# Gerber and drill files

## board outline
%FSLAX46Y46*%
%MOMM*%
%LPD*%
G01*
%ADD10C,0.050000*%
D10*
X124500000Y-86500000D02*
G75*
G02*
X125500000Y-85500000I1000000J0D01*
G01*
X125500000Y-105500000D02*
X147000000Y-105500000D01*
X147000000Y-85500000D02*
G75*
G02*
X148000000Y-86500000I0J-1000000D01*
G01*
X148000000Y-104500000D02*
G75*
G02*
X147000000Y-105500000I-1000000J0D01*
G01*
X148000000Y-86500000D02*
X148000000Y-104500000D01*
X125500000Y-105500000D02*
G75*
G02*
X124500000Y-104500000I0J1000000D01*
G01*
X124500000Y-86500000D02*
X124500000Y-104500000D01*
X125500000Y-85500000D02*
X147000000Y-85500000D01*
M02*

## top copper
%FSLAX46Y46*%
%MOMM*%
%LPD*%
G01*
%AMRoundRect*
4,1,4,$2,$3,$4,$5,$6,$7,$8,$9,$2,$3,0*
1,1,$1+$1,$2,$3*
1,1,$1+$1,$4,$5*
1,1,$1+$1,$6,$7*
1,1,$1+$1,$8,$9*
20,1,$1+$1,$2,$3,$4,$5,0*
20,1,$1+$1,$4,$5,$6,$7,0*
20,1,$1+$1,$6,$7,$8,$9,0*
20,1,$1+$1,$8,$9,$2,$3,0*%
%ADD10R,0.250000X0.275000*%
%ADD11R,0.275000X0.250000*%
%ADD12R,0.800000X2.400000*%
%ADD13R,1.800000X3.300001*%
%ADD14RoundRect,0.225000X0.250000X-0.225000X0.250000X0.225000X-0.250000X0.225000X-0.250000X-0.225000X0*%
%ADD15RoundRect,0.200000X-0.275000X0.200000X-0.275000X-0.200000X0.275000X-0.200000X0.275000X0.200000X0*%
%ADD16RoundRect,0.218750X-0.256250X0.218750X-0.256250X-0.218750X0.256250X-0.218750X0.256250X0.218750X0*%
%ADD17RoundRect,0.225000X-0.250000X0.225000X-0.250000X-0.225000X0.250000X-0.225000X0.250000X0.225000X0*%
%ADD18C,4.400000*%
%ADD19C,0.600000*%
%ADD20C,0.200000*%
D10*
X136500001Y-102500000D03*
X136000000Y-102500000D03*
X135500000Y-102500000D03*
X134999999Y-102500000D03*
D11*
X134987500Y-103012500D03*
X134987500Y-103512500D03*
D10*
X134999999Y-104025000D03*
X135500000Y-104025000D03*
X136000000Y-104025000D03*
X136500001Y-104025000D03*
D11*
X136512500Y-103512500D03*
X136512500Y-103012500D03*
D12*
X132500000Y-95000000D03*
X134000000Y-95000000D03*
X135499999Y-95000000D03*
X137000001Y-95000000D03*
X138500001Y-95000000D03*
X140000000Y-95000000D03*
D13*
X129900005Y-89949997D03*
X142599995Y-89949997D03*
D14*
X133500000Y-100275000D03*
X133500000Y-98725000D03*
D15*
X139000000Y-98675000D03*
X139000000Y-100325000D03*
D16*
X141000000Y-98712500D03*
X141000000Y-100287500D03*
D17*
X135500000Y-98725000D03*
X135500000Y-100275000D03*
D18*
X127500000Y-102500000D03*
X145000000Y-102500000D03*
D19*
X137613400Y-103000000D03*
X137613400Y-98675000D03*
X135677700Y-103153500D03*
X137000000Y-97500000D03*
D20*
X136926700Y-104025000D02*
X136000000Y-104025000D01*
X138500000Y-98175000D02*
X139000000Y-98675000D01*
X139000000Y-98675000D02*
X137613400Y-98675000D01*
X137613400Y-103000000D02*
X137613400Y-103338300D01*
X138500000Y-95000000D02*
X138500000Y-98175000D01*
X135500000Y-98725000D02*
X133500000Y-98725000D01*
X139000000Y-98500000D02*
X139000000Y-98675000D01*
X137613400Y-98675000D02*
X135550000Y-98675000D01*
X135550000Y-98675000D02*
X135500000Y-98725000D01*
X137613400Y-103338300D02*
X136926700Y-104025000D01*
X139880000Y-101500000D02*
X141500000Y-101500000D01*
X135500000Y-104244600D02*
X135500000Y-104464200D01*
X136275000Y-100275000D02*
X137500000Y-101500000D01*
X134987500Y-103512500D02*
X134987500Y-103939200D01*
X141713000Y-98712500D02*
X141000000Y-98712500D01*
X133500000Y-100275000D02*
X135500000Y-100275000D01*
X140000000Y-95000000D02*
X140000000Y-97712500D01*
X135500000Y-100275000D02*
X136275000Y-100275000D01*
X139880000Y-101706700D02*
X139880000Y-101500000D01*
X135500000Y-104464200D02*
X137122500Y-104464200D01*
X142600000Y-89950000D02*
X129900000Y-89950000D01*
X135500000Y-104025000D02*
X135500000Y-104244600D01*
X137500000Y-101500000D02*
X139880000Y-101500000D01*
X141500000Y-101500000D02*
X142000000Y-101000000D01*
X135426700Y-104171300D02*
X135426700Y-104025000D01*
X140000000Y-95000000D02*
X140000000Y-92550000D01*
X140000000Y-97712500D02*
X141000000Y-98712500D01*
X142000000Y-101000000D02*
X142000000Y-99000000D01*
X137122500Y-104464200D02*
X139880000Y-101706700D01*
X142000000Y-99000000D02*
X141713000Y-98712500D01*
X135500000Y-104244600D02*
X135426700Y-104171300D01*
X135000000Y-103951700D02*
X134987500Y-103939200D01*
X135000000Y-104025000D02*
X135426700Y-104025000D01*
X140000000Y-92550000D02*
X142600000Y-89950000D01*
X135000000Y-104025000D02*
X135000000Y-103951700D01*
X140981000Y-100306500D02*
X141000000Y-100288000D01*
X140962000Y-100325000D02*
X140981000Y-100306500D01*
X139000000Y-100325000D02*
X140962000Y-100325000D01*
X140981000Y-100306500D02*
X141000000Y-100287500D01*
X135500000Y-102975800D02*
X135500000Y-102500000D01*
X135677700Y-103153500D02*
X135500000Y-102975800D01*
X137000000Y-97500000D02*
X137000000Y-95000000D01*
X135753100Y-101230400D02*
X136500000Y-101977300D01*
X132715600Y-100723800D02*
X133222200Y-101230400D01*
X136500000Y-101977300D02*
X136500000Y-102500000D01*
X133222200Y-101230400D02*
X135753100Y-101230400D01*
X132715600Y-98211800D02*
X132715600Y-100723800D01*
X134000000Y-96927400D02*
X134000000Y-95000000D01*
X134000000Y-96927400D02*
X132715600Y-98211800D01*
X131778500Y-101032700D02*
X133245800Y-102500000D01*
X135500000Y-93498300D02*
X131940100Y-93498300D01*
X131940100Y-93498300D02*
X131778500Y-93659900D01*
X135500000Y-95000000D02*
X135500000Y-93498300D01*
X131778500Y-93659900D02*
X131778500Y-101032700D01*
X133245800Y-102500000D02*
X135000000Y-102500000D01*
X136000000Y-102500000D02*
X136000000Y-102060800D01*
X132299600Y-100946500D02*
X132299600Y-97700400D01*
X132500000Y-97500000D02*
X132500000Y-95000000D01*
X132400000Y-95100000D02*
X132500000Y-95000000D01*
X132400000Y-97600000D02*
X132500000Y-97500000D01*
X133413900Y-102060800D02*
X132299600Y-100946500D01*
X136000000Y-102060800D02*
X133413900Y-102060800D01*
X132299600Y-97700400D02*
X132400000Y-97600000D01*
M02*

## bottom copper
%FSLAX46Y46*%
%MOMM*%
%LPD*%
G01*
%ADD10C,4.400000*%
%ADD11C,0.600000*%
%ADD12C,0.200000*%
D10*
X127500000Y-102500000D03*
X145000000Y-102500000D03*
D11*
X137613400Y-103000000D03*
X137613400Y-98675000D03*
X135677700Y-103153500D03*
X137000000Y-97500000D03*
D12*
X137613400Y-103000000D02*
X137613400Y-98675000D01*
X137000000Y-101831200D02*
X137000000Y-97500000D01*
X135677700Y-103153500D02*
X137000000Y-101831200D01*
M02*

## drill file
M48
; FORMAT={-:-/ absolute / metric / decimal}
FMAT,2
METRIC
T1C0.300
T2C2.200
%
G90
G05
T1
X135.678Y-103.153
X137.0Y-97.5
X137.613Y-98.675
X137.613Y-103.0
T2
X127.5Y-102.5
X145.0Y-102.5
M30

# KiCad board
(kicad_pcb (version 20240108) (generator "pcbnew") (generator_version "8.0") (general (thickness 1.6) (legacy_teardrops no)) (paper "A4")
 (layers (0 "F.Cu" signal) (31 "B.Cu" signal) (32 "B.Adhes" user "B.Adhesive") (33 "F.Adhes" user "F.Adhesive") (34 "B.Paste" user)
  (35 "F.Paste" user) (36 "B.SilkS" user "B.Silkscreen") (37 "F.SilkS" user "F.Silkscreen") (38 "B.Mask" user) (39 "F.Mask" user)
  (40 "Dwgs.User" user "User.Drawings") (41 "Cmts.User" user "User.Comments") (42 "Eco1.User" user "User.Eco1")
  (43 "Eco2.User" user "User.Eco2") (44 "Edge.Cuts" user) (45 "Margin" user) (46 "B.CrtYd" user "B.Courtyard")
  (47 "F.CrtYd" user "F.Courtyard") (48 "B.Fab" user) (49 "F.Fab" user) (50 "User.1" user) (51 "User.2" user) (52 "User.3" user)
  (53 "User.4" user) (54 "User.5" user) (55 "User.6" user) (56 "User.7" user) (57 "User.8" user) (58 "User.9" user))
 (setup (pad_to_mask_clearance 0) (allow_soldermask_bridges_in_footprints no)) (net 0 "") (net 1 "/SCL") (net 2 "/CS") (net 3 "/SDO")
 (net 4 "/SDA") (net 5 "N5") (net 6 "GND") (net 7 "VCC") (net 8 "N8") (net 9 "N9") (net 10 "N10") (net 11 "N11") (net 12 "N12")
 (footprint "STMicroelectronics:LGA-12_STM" (layer "F.Cu") (at 135.75 103.2625 -90)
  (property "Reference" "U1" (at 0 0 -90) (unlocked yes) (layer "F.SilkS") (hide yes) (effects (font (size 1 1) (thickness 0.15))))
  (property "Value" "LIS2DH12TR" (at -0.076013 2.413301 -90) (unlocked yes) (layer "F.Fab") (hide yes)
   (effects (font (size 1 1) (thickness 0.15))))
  (pad "1" smd rect (at -0.7625 -0.750001) (size 0.25 0.275) (layers "F.Cu" "F.Paste" "F.Mask") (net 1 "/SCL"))
  (pad "2" smd rect (at -0.7625 -0.25) (size 0.25 0.275) (layers "F.Cu" "F.Paste" "F.Mask") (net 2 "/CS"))
  (pad "3" smd rect (at -0.7625 0.25) (size 0.25 0.275) (layers "F.Cu" "F.Paste" "F.Mask") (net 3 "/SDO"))
  (pad "4" smd rect (at -0.7625 0.750001) (size 0.25 0.275) (layers "F.Cu" "F.Paste" "F.Mask") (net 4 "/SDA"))
  (pad "5" smd rect (at -0.25 0.7625 270) (size 0.25 0.275) (layers "F.Cu" "F.Paste" "F.Mask") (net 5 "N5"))
  (pad "6" smd rect (at 0.25 0.7625 270) (size 0.25 0.275) (layers "F.Cu" "F.Paste" "F.Mask") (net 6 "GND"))
  (pad "7" smd rect (at 0.7625 0.750001) (size 0.25 0.275) (layers "F.Cu" "F.Paste" "F.Mask") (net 6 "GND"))
  (pad "8" smd rect (at 0.7625 0.25) (size 0.25 0.275) (layers "F.Cu" "F.Paste" "F.Mask") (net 6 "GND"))
  (pad "9" smd rect (at 0.7625 -0.25) (size 0.25 0.275) (layers "F.Cu" "F.Paste" "F.Mask") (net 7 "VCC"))
  (pad "10" smd rect (at 0.7625 -0.750001) (size 0.25 0.275) (layers "F.Cu" "F.Paste" "F.Mask") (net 7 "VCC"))
  (pad "11" smd rect (at 0.25 -0.7625 270) (size 0.25 0.275) (layers "F.Cu" "F.Paste" "F.Mask") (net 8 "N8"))
  (pad "12" smd rect (at -0.25 -0.7625 270) (size 0.25 0.275) (layers "F.Cu" "F.Paste" "F.Mask") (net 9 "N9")))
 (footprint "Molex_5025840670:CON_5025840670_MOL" (layer "F.Cu") (at 132.5 95)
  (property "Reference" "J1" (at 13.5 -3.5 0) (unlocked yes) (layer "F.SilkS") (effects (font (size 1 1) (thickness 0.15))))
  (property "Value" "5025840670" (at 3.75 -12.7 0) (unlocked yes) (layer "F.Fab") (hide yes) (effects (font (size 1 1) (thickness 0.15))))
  (pad "1" smd rect (at 0 0) (size 0.8 2.4) (layers "F.Cu" "F.Paste" "F.Mask") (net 2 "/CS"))
  (pad "2" smd rect (at 1.5 0) (size 0.8 2.4) (layers "F.Cu" "F.Paste" "F.Mask") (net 1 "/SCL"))
  (pad "3" smd rect (at 2.999999 0) (size 0.8 2.4) (layers "F.Cu" "F.Paste" "F.Mask") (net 4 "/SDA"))
  (pad "4" smd rect (at 4.500001 0) (size 0.8 2.4) (layers "F.Cu" "F.Paste" "F.Mask") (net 3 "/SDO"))
  (pad "5" smd rect (at 6.000001 0) (size 0.8 2.4) (layers "F.Cu" "F.Paste" "F.Mask") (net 7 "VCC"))
  (pad "6" smd rect (at 7.5 0) (size 0.8 2.4) (layers "F.Cu" "F.Paste" "F.Mask") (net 6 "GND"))
  (pad "7" smd rect (at -2.599995 -5.050003) (size 1.8 3.300001) (layers "F.Cu" "F.Paste" "F.Mask") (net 6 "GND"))
  (pad "8" smd rect (at 10.099995 -5.050003) (size 1.8 3.300001) (layers "F.Cu" "F.Paste" "F.Mask") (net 6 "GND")))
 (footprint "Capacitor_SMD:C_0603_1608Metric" (layer "F.Cu") (at 133.5 99.5 90)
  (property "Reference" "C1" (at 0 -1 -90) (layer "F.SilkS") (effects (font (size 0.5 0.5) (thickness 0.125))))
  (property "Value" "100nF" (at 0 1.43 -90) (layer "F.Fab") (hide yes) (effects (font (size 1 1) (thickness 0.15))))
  (pad "1" smd roundrect (at -0.775 0 90) (size 0.9 0.95) (layers "F.Cu" "F.Paste" "F.Mask") (roundrect_rratio 0.25) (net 6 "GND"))
  (pad "2" smd roundrect (at 0.775 0 90) (size 0.9 0.95) (layers "F.Cu" "F.Paste" "F.Mask") (roundrect_rratio 0.25) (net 7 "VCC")))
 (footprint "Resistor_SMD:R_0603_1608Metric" (layer "F.Cu") (at 139 99.5 -90)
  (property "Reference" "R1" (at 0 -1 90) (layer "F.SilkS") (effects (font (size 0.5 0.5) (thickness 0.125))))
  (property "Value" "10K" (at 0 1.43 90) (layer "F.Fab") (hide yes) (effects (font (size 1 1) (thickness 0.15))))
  (pad "1" smd roundrect (at -0.825 0 270) (size 0.8 0.95) (layers "F.Cu" "F.Paste" "F.Mask") (roundrect_rratio 0.25) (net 7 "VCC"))
  (pad "2" smd roundrect (at 0.825 0 270) (size 0.8 0.95) (layers "F.Cu" "F.Paste" "F.Mask") (roundrect_rratio 0.25) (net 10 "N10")))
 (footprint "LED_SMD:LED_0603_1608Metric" (layer "F.Cu") (at 141 99.5 -90)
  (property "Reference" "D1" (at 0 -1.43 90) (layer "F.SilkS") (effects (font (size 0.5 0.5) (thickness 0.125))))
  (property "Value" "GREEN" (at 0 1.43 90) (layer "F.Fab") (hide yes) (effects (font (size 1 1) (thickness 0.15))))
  (pad "1" smd roundrect (at -0.7875 0 270) (size 0.875 0.95) (layers "F.Cu" "F.Paste" "F.Mask") (roundrect_rratio 0.25) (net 6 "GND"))
  (pad "2" smd roundrect (at 0.7875 0 270) (size 0.875 0.95) (layers "F.Cu" "F.Paste" "F.Mask") (roundrect_rratio 0.25) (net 10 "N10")))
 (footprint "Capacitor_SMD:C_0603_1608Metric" (layer "F.Cu") (at 135.5 99.5 -90)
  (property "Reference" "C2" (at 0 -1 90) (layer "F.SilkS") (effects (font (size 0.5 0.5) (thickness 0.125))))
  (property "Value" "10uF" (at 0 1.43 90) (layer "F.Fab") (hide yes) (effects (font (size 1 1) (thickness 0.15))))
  (pad "1" smd roundrect (at -0.775 0 270) (size 0.9 0.95) (layers "F.Cu" "F.Paste" "F.Mask") (roundrect_rratio 0.25) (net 7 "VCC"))
  (pad "2" smd roundrect (at 0.775 0 270) (size 0.9 0.95) (layers "F.Cu" "F.Paste" "F.Mask") (roundrect_rratio 0.25) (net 6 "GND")))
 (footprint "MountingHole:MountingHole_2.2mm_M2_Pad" (layer "F.Cu") (at 127.5 102.5)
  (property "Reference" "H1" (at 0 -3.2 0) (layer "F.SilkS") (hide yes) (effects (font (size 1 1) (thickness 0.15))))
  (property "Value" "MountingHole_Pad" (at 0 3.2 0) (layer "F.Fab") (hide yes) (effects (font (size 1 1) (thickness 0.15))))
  (pad "1" thru_hole circle (at 0 0) (size 4.4 4.4) (drill 2.2) (layers "*.Cu" "*.Mask") (remove_unused_layers no) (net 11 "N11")))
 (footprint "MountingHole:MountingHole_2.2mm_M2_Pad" (layer "F.Cu") (at 145 102.5)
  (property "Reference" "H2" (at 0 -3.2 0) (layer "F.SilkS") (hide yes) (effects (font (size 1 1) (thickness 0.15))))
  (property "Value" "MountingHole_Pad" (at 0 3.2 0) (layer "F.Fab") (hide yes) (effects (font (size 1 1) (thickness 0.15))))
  (pad "1" thru_hole circle (at 0 0) (size 4.4 4.4) (drill 2.2) (layers "*.Cu" "*.Mask") (remove_unused_layers no) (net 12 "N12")))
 (gr_arc (start 124.5 86.5) (mid 124.792893 85.792893) (end 125.5 85.5) (stroke (width 0.05) (type default)) (layer "Edge.Cuts"))
 (gr_line (start 125.5 105.5) (end 147 105.5) (stroke (width 0.05) (type default)) (layer "Edge.Cuts"))
 (gr_arc (start 147 85.5) (mid 147.707107 85.792893) (end 148 86.5) (stroke (width 0.05) (type default)) (layer "Edge.Cuts"))
 (gr_arc (start 148 104.5) (mid 147.707107 105.207107) (end 147 105.5) (stroke (width 0.05) (type default)) (layer "Edge.Cuts"))
 (gr_line (start 148 86.5) (end 148 104.5) (stroke (width 0.05) (type default)) (layer "Edge.Cuts"))
 (gr_arc (start 125.5 105.5) (mid 124.792893 105.207107) (end 124.5 104.5) (stroke (width 0.05) (type default)) (layer "Edge.Cuts"))
 (gr_line (start 124.5 86.5) (end 124.5 104.5) (stroke (width 0.05) (type default)) (layer "Edge.Cuts"))
 (gr_line (start 125.5 85.5) (end 147 85.5) (stroke (width 0.05) (type default)) (layer "Edge.Cuts"))
 (segment (start 136.9267 104.025) (end 136 104.025) (width 0.2) (layer "F.Cu") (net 7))
 (segment (start 138.5 98.175) (end 139 98.675) (width 0.2) (layer "F.Cu") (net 7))
 (segment (start 139 98.675) (end 137.6134 98.675) (width 0.2) (layer "F.Cu") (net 7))
 (segment (start 137.6134 103) (end 137.6134 103.3383) (width 0.2) (layer "F.Cu") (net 7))
 (segment (start 138.5 95) (end 138.5 98.175) (width 0.2) (layer "F.Cu") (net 7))
 (segment (start 135.5 98.725) (end 133.5 98.725) (width 0.2) (layer "F.Cu") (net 7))
 (segment (start 139 98.5) (end 139 98.675) (width 0.2) (layer "F.Cu") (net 7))
 (segment (start 137.6134 98.675) (end 135.55 98.675) (width 0.2) (layer "F.Cu") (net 7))
 (segment (start 135.55 98.675) (end 135.5 98.725) (width 0.2) (layer "F.Cu") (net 7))
 (segment (start 137.6134 103.3383) (end 136.9267 104.025) (width 0.2) (layer "F.Cu") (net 7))
 (via (at 137.6134 103) (size 0.6) (drill 0.3) (layers "F.Cu" "B.Cu") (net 7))
 (via (at 137.6134 98.675) (size 0.6) (drill 0.3) (layers "F.Cu" "B.Cu") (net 7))
 (segment (start 137.6134 103) (end 137.6134 98.675) (width 0.2) (layer "B.Cu") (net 7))
 (segment (start 139.88 101.5) (end 141.5 101.5) (width 0.2) (layer "F.Cu") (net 6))
 (segment (start 135.5 104.2446) (end 135.5 104.4642) (width 0.2) (layer "F.Cu") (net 6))
 (segment (start 136.275 100.275) (end 137.5 101.5) (width 0.2) (layer "F.Cu") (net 6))
 (segment (start 134.9875 103.5125) (end 134.9875 103.9392) (width 0.2) (layer "F.Cu") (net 6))
 (segment (start 141.713 98.7125) (end 141 98.7125) (width 0.2) (layer "F.Cu") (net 6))
 (segment (start 133.5 100.275) (end 135.5 100.275) (width 0.2) (layer "F.Cu") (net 6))
 (segment (start 140 95) (end 140 97.7125) (width 0.2) (layer "F.Cu") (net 6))
 (segment (start 135.5 100.275) (end 136.275 100.275) (width 0.2) (layer "F.Cu") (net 6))
 (segment (start 139.88 101.7067) (end 139.88 101.5) (width 0.2) (layer "F.Cu") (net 6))
 (segment (start 135.5 104.4642) (end 137.1225 104.4642) (width 0.2) (layer "F.Cu") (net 6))
 (segment (start 142.6 89.95) (end 129.9 89.95) (width 0.2) (layer "F.Cu") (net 6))
 (segment (start 135.5 104.025) (end 135.5 104.2446) (width 0.2) (layer "F.Cu") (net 6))
 (segment (start 137.5 101.5) (end 139.88 101.5) (width 0.2) (layer "F.Cu") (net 6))
 (segment (start 141.5 101.5) (end 142 101) (width 0.2) (layer "F.Cu") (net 6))
 (segment (start 135.4267 104.1713) (end 135.4267 104.025) (width 0.2) (layer "F.Cu") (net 6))
 (segment (start 140 95) (end 140 92.55) (width 0.2) (layer "F.Cu") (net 6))
 (segment (start 140 97.7125) (end 141 98.7125) (width 0.2) (layer "F.Cu") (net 6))
 (segment (start 142 101) (end 142 99) (width 0.2) (layer "F.Cu") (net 6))
 (segment (start 137.1225 104.4642) (end 139.88 101.7067) (width 0.2) (layer "F.Cu") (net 6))
 (segment (start 142 99) (end 141.713 98.7125) (width 0.2) (layer "F.Cu") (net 6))
 (segment (start 135.5 104.2446) (end 135.4267 104.1713) (width 0.2) (layer "F.Cu") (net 6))
 (segment (start 135 103.9517) (end 134.9875 103.9392) (width 0.2) (layer "F.Cu") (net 6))
 (segment (start 135 104.025) (end 135.4267 104.025) (width 0.2) (layer "F.Cu") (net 6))
 (segment (start 140 92.55) (end 142.6 89.95) (width 0.2) (layer "F.Cu") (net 6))
 (segment (start 135 104.025) (end 135 103.9517) (width 0.2) (layer "F.Cu") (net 6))
 (segment (start 140.981 100.3065) (end 141 100.288) (width 0.2) (layer "F.Cu") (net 10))
 (segment (start 140.962 100.325) (end 140.981 100.3065) (width 0.2) (layer "F.Cu") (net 10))
 (segment (start 139 100.325) (end 140.962 100.325) (width 0.2) (layer "F.Cu") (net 10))
 (segment (start 140.981 100.3065) (end 141 100.2875) (width 0.2) (layer "F.Cu") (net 10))
 (segment (start 135.5 102.9758) (end 135.5 102.5) (width 0.2) (layer "F.Cu") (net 3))
 (segment (start 135.6777 103.1535) (end 135.5 102.9758) (width 0.2) (layer "F.Cu") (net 3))
 (segment (start 137 97.5) (end 137 95) (width 0.2) (layer "F.Cu") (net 3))
 (via (at 135.6777 103.1535) (size 0.6) (drill 0.3) (layers "F.Cu" "B.Cu") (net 3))
 (via (at 137 97.5) (size 0.6) (drill 0.3) (layers "F.Cu" "B.Cu") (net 3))
 (segment (start 137 101.8312) (end 137 97.5) (width 0.2) (layer "B.Cu") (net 3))
 (segment (start 135.6777 103.1535) (end 137 101.8312) (width 0.2) (layer "B.Cu") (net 3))
 (segment (start 135.7531 101.2304) (end 136.5 101.9773) (width 0.2) (layer "F.Cu") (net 1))
 (segment (start 132.7156 100.7238) (end 133.2222 101.2304) (width 0.2) (layer "F.Cu") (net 1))
 (segment (start 136.5 101.9773) (end 136.5 102.5) (width 0.2) (layer "F.Cu") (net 1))
 (segment (start 133.2222 101.2304) (end 135.7531 101.2304) (width 0.2) (layer "F.Cu") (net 1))
 (segment (start 132.7156 98.2118) (end 132.7156 100.7238) (width 0.2) (layer "F.Cu") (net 1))
 (segment (start 134 96.9274) (end 134 95) (width 0.2) (layer "F.Cu") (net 1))
 (segment (start 134 96.9274) (end 132.7156 98.2118) (width 0.2) (layer "F.Cu") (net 1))
 (segment (start 131.7785 101.0327) (end 133.2458 102.5) (width 0.2) (layer "F.Cu") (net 4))
 (segment (start 135.5 93.4983) (end 131.9401 93.4983) (width 0.2) (layer "F.Cu") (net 4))
 (segment (start 131.9401 93.4983) (end 131.7785 93.6599) (width 0.2) (layer "F.Cu") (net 4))
 (segment (start 135.5 95) (end 135.5 93.4983) (width 0.2) (layer "F.Cu") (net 4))
 (segment (start 131.7785 93.6599) (end 131.7785 101.0327) (width 0.2) (layer "F.Cu") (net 4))
 (segment (start 133.2458 102.5) (end 135 102.5) (width 0.2) (layer "F.Cu") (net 4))
 (segment (start 136 102.5) (end 136 102.0608) (width 0.2) (layer "F.Cu") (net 2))
 (segment (start 132.2996 100.9465) (end 132.2996 97.7004) (width 0.2) (layer "F.Cu") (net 2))
 (segment (start 132.5 97.5) (end 132.5 95) (width 0.2) (layer "F.Cu") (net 2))
 (segment (start 132.4 95.1) (end 132.5 95) (width 0.2) (layer "F.Cu") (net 2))
 (segment (start 132.4 97.6) (end 132.5 97.5) (width 0.2) (layer "F.Cu") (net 2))
 (segment (start 133.4139 102.0608) (end 132.2996 100.9465) (width 0.2) (layer "F.Cu") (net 2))
 (segment (start 136 102.0608) (end 133.4139 102.0608) (width 0.2) (layer "F.Cu") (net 2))
 (segment (start 132.2996 97.7004) (end 132.4 97.6) (width 0.2) (layer "F.Cu") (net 2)))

